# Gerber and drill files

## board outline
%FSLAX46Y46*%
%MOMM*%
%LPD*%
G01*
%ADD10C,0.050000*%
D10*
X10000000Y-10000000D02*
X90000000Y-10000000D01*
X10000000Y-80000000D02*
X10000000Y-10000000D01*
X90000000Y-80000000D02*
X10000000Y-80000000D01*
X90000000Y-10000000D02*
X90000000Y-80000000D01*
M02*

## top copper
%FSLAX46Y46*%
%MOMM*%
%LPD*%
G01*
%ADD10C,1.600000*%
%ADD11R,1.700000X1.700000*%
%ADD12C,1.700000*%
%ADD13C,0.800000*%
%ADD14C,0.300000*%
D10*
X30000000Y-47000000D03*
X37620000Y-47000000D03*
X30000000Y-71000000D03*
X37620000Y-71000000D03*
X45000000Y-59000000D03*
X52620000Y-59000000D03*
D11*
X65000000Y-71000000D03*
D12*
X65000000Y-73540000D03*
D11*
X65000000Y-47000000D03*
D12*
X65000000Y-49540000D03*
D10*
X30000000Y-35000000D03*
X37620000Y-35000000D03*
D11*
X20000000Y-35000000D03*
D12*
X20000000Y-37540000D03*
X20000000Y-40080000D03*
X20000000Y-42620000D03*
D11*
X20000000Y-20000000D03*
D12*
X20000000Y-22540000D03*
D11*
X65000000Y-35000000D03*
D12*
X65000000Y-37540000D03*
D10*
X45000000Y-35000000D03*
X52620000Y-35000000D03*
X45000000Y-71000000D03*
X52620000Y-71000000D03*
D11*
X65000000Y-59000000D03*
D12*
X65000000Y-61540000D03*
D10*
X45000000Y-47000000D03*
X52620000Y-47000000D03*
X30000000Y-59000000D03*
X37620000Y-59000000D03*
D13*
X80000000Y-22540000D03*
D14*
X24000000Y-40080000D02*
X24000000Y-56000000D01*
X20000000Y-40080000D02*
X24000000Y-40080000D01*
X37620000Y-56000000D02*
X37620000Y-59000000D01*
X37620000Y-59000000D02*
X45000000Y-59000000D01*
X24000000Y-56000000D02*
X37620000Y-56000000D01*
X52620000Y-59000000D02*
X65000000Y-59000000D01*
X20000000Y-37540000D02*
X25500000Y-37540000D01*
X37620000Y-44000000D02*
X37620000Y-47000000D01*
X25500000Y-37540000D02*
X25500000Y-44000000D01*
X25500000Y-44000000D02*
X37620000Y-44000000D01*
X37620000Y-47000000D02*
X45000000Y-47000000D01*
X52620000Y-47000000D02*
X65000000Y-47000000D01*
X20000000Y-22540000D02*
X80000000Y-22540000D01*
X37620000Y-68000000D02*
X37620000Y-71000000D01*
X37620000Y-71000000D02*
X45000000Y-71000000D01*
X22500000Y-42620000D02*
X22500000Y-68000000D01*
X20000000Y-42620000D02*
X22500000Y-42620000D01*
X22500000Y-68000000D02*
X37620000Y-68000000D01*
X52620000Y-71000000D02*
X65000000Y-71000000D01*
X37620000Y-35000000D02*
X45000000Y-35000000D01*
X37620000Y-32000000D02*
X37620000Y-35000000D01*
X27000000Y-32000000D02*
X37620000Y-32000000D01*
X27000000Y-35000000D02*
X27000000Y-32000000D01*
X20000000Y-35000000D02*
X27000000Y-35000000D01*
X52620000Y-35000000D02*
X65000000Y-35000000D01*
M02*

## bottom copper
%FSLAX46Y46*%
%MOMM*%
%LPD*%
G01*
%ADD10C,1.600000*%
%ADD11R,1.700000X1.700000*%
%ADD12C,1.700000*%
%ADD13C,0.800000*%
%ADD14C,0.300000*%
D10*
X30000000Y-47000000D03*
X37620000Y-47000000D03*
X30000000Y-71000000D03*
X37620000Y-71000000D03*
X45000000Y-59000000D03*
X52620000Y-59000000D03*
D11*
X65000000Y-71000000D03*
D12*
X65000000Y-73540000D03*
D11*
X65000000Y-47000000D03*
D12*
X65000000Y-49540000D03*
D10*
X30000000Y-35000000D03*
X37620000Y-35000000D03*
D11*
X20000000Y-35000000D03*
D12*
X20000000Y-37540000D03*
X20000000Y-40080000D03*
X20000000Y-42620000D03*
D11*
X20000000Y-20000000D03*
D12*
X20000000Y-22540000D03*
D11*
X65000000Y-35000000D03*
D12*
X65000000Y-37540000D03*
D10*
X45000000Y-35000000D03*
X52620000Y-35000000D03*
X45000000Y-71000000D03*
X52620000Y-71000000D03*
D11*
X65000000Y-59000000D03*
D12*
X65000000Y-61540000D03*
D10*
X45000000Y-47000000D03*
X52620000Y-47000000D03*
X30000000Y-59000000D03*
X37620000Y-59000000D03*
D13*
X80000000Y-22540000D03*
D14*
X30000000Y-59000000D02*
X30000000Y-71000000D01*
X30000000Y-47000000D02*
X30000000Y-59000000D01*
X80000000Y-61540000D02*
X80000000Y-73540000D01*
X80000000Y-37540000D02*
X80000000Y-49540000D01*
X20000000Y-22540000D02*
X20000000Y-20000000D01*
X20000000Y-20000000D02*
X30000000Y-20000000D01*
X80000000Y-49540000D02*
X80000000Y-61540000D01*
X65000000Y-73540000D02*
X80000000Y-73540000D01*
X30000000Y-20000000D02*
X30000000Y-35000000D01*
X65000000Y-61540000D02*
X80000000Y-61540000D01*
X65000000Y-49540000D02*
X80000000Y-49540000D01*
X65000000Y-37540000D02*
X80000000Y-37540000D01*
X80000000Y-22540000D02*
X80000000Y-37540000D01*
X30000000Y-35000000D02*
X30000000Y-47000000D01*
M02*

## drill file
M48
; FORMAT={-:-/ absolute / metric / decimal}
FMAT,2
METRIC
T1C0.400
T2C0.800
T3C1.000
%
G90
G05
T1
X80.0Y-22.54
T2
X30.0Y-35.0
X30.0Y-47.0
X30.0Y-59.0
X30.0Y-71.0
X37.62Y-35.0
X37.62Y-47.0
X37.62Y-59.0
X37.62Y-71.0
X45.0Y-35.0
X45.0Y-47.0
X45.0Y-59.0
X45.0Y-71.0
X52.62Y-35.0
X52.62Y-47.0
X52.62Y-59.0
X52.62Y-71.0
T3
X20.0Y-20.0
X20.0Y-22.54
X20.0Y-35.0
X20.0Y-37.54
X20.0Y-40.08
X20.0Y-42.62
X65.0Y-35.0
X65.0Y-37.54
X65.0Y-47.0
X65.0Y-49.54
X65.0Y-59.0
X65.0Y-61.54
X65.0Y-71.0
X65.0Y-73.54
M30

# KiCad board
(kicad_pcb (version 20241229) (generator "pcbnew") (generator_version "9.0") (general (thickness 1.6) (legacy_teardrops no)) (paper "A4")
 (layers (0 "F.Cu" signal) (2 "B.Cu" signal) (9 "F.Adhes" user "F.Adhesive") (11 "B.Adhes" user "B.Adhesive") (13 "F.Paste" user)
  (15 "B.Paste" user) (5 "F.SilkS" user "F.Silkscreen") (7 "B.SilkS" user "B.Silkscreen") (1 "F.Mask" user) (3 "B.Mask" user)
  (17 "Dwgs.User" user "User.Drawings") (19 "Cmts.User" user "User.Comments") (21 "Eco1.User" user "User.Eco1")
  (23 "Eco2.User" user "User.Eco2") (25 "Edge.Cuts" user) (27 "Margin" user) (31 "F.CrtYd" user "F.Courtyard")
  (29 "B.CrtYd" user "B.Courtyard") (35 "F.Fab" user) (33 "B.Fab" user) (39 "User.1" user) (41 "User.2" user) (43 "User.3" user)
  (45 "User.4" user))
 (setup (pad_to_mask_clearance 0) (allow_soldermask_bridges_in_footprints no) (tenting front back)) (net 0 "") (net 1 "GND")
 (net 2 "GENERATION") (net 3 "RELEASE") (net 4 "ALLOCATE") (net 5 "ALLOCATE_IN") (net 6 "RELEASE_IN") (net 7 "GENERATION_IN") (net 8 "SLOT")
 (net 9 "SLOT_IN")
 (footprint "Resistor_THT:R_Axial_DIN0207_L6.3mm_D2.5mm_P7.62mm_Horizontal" (layer "F.Cu") (at 30 47)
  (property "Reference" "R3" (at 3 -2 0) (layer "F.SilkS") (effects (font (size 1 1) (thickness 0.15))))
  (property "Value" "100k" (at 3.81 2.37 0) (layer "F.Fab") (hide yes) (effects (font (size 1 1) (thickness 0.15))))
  (pad "1" thru_hole circle (at 0 0) (size 1.6 1.6) (drill 0.8) (layers "*.Cu" "*.Mask") (remove_unused_layers no) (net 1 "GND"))
  (pad "2" thru_hole circle (at 7.62 0) (size 1.6 1.6) (drill 0.8) (layers "*.Cu" "*.Mask") (remove_unused_layers no) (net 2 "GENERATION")))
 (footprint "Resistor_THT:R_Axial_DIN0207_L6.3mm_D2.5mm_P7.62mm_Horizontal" (layer "F.Cu") (at 30 71)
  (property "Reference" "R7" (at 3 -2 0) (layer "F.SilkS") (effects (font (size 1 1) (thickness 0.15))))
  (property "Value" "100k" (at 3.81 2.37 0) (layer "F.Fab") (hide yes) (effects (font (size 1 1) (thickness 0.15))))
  (pad "1" thru_hole circle (at 0 0) (size 1.6 1.6) (drill 0.8) (layers "*.Cu" "*.Mask") (remove_unused_layers no) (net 1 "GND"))
  (pad "2" thru_hole circle (at 7.62 0) (size 1.6 1.6) (drill 0.8) (layers "*.Cu" "*.Mask") (remove_unused_layers no) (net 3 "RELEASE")))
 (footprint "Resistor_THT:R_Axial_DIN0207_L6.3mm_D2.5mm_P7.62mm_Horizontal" (layer "F.Cu") (at 45 59)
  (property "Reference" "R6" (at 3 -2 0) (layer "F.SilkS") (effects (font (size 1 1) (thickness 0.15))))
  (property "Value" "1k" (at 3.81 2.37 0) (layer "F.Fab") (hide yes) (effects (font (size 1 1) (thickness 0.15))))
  (pad "1" thru_hole circle (at 0 0) (size 1.6 1.6) (drill 0.8) (layers "*.Cu" "*.Mask") (remove_unused_layers no) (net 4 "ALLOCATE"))
  (pad "2" thru_hole circle (at 7.62 0) (size 1.6 1.6) (drill 0.8) (layers "*.Cu" "*.Mask") (remove_unused_layers no) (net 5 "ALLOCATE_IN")))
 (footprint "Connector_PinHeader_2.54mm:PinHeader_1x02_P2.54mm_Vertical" (layer "F.Cu") (at 65 71)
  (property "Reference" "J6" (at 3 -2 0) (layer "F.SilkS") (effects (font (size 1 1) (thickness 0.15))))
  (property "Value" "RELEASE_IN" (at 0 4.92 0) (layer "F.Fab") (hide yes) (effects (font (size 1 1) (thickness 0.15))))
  (pad "1" thru_hole rect (at 0 0) (size 1.7 1.7) (drill 1) (layers "*.Cu" "*.Mask") (remove_unused_layers no) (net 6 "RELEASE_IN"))
  (pad "2" thru_hole circle (at 0 2.54) (size 1.7 1.7) (drill 1) (layers "*.Cu" "*.Mask") (remove_unused_layers no) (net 1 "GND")))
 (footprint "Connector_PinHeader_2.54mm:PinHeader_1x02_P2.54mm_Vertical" (layer "F.Cu") (at 65 47)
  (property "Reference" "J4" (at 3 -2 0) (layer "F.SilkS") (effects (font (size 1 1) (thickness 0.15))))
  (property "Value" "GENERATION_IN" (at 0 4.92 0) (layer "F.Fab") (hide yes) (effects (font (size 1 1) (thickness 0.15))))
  (pad "1" thru_hole rect (at 0 0) (size 1.7 1.7) (drill 1) (layers "*.Cu" "*.Mask") (remove_unused_layers no) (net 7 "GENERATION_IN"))
  (pad "2" thru_hole circle (at 0 2.54) (size 1.7 1.7) (drill 1) (layers "*.Cu" "*.Mask") (remove_unused_layers no) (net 1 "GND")))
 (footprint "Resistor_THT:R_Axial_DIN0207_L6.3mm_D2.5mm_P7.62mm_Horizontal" (layer "F.Cu") (at 30 35)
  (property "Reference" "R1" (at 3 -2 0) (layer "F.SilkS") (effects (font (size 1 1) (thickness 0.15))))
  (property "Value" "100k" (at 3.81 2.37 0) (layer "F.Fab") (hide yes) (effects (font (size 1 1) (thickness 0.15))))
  (pad "1" thru_hole circle (at 0 0) (size 1.6 1.6) (drill 0.8) (layers "*.Cu" "*.Mask") (remove_unused_layers no) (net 1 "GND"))
  (pad "2" thru_hole circle (at 7.62 0) (size 1.6 1.6) (drill 0.8) (layers "*.Cu" "*.Mask") (remove_unused_layers no) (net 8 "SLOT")))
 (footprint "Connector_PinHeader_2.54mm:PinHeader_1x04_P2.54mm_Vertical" (layer "F.Cu") (at 20 35)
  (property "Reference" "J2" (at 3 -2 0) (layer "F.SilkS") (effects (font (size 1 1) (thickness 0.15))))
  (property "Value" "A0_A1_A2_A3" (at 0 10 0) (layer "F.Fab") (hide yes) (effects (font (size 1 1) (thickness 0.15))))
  (pad "1" thru_hole rect (at 0 0) (size 1.7 1.7) (drill 1) (layers "*.Cu" "*.Mask") (remove_unused_layers no) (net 8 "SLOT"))
  (pad "2" thru_hole circle (at 0 2.54) (size 1.7 1.7) (drill 1) (layers "*.Cu" "*.Mask") (remove_unused_layers no) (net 2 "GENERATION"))
  (pad "3" thru_hole circle (at 0 5.08) (size 1.7 1.7) (drill 1) (layers "*.Cu" "*.Mask") (remove_unused_layers no) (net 4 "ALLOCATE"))
  (pad "4" thru_hole circle (at 0 7.62) (size 1.7 1.7) (drill 1) (layers "*.Cu" "*.Mask") (remove_unused_layers no) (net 3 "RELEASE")))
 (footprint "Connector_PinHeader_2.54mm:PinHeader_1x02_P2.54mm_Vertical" (layer "F.Cu") (at 20 20)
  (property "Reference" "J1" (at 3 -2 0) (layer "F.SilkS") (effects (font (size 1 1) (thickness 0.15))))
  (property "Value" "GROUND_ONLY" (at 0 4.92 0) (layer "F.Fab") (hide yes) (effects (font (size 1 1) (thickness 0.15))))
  (pad "1" thru_hole rect (at 0 0) (size 1.7 1.7) (drill 1) (layers "*.Cu" "*.Mask") (remove_unused_layers no) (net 1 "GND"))
  (pad "2" thru_hole circle (at 0 2.54) (size 1.7 1.7) (drill 1) (layers "*.Cu" "*.Mask") (remove_unused_layers no) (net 1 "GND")))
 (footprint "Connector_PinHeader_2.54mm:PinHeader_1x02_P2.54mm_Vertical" (layer "F.Cu") (at 65 35)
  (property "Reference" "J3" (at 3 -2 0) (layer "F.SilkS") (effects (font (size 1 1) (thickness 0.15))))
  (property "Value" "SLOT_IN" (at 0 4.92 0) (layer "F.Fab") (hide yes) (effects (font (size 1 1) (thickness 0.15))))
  (pad "1" thru_hole rect (at 0 0) (size 1.7 1.7) (drill 1) (layers "*.Cu" "*.Mask") (remove_unused_layers no) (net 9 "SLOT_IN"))
  (pad "2" thru_hole circle (at 0 2.54) (size 1.7 1.7) (drill 1) (layers "*.Cu" "*.Mask") (remove_unused_layers no) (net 1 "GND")))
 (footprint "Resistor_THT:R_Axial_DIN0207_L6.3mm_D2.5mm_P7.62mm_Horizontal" (layer "F.Cu") (at 45 35)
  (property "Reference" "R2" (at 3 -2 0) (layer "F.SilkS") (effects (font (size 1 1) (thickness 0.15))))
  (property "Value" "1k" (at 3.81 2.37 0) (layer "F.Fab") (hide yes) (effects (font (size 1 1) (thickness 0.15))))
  (pad "1" thru_hole circle (at 0 0) (size 1.6 1.6) (drill 0.8) (layers "*.Cu" "*.Mask") (remove_unused_layers no) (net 8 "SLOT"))
  (pad "2" thru_hole circle (at 7.62 0) (size 1.6 1.6) (drill 0.8) (layers "*.Cu" "*.Mask") (remove_unused_layers no) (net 9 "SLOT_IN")))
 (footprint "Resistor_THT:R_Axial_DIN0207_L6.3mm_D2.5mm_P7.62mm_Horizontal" (layer "F.Cu") (at 45 71)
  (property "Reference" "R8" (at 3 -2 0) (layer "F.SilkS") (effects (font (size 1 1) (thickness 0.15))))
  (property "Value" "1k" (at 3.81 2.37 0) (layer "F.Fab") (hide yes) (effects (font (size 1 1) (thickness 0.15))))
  (pad "1" thru_hole circle (at 0 0) (size 1.6 1.6) (drill 0.8) (layers "*.Cu" "*.Mask") (remove_unused_layers no) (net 3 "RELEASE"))
  (pad "2" thru_hole circle (at 7.62 0) (size 1.6 1.6) (drill 0.8) (layers "*.Cu" "*.Mask") (remove_unused_layers no) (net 6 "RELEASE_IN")))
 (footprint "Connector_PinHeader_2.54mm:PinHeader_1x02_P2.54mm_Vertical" (layer "F.Cu") (at 65 59)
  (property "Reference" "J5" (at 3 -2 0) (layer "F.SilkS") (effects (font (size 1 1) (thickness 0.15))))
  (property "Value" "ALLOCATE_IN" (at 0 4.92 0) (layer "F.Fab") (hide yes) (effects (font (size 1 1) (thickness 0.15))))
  (pad "1" thru_hole rect (at 0 0) (size 1.7 1.7) (drill 1) (layers "*.Cu" "*.Mask") (remove_unused_layers no) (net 5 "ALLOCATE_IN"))
  (pad "2" thru_hole circle (at 0 2.54) (size 1.7 1.7) (drill 1) (layers "*.Cu" "*.Mask") (remove_unused_layers no) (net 1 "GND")))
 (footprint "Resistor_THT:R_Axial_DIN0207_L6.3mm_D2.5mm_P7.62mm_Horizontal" (layer "F.Cu") (at 45 47)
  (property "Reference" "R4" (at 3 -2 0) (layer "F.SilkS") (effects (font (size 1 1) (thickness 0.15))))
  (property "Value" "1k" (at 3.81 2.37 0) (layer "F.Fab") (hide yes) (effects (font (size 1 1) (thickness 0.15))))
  (pad "1" thru_hole circle (at 0 0) (size 1.6 1.6) (drill 0.8) (layers "*.Cu" "*.Mask") (remove_unused_layers no) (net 2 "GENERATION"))
  (pad "2" thru_hole circle (at 7.62 0) (size 1.6 1.6) (drill 0.8) (layers "*.Cu" "*.Mask") (remove_unused_layers no)
   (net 7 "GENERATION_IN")))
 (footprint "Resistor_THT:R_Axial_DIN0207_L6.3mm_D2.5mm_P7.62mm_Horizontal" (layer "F.Cu") (at 30 59)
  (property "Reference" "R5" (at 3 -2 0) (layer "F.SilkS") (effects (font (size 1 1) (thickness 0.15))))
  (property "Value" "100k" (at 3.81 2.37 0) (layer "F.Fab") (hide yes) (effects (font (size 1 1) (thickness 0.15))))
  (pad "1" thru_hole circle (at 0 0) (size 1.6 1.6) (drill 0.8) (layers "*.Cu" "*.Mask") (remove_unused_layers no) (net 1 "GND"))
  (pad "2" thru_hole circle (at 7.62 0) (size 1.6 1.6) (drill 0.8) (layers "*.Cu" "*.Mask") (remove_unused_layers no) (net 4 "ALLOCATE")))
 (gr_line (start 10 10) (end 90 10) (stroke (width 0.05) (type default)) (layer "Edge.Cuts"))
 (gr_line (start 10 80) (end 10 10) (stroke (width 0.05) (type default)) (layer "Edge.Cuts"))
 (gr_line (start 90 80) (end 10 80) (stroke (width 0.05) (type default)) (layer "Edge.Cuts"))
 (gr_line (start 90 10) (end 90 80) (stroke (width 0.05) (type default)) (layer "Edge.Cuts"))
 (segment (start 24 40.08) (end 24 56) (width 0.3) (layer "F.Cu") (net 4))
 (segment (start 20 40.08) (end 24 40.08) (width 0.3) (layer "F.Cu") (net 4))
 (segment (start 37.62 56) (end 37.62 59) (width 0.3) (layer "F.Cu") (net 4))
 (segment (start 37.62 59) (end 45 59) (width 0.3) (layer "F.Cu") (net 4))
 (segment (start 24 56) (end 37.62 56) (width 0.3) (layer "F.Cu") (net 4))
 (segment (start 52.62 59) (end 65 59) (width 0.3) (layer "F.Cu") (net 5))
 (segment (start 20 37.54) (end 25.5 37.54) (width 0.3) (layer "F.Cu") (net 2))
 (segment (start 37.62 44) (end 37.62 47) (width 0.3) (layer "F.Cu") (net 2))
 (segment (start 25.5 37.54) (end 25.5 44) (width 0.3) (layer "F.Cu") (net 2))
 (segment (start 25.5 44) (end 37.62 44) (width 0.3) (layer "F.Cu") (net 2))
 (segment (start 37.62 47) (end 45 47) (width 0.3) (layer "F.Cu") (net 2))
 (segment (start 52.62 47) (end 65 47) (width 0.3) (layer "F.Cu") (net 7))
 (segment (start 20 22.54) (end 80 22.54) (width 0.3) (layer "F.Cu") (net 1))
 (via (at 80 22.54) (size 0.8) (drill 0.4) (layers "F.Cu" "B.Cu") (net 1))
 (segment (start 30 59) (end 30 71) (width 0.3) (layer "B.Cu") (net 1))
 (segment (start 30 47) (end 30 59) (width 0.3) (layer "B.Cu") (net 1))
 (segment (start 80 61.54) (end 80 73.54) (width 0.3) (layer "B.Cu") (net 1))
 (segment (start 80 37.54) (end 80 49.54) (width 0.3) (layer "B.Cu") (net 1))
 (segment (start 20 22.54) (end 20 20) (width 0.3) (layer "B.Cu") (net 1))
 (segment (start 20 20) (end 30 20) (width 0.3) (layer "B.Cu") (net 1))
 (segment (start 80 49.54) (end 80 61.54) (width 0.3) (layer "B.Cu") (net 1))
 (segment (start 65 73.54) (end 80 73.54) (width 0.3) (layer "B.Cu") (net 1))
 (segment (start 30 20) (end 30 35) (width 0.3) (layer "B.Cu") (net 1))
 (segment (start 65 61.54) (end 80 61.54) (width 0.3) (layer "B.Cu") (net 1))
 (segment (start 65 49.54) (end 80 49.54) (width 0.3) (layer "B.Cu") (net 1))
 (segment (start 65 37.54) (end 80 37.54) (width 0.3) (layer "B.Cu") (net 1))
 (segment (start 80 22.54) (end 80 37.54) (width 0.3) (layer "B.Cu") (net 1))
 (segment (start 30 35) (end 30 47) (width 0.3) (layer "B.Cu") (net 1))
 (segment (start 37.62 68) (end 37.62 71) (width 0.3) (layer "F.Cu") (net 3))
 (segment (start 37.62 71) (end 45 71) (width 0.3) (layer "F.Cu") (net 3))
 (segment (start 22.5 42.62) (end 22.5 68) (width 0.3) (layer "F.Cu") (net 3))
 (segment (start 20 42.62) (end 22.5 42.62) (width 0.3) (layer "F.Cu") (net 3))
 (segment (start 22.5 68) (end 37.62 68) (width 0.3) (layer "F.Cu") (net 3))
 (segment (start 52.62 71) (end 65 71) (width 0.3) (layer "F.Cu") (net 6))
 (segment (start 37.62 35) (end 45 35) (width 0.3) (layer "F.Cu") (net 8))
 (segment (start 37.62 32) (end 37.62 35) (width 0.3) (layer "F.Cu") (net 8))
 (segment (start 27 32) (end 37.62 32) (width 0.3) (layer "F.Cu") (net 8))
 (segment (start 27 35) (end 27 32) (width 0.3) (layer "F.Cu") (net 8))
 (segment (start 20 35) (end 27 35) (width 0.3) (layer "F.Cu") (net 8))
 (segment (start 52.62 35) (end 65 35) (width 0.3) (layer "F.Cu") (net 9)))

